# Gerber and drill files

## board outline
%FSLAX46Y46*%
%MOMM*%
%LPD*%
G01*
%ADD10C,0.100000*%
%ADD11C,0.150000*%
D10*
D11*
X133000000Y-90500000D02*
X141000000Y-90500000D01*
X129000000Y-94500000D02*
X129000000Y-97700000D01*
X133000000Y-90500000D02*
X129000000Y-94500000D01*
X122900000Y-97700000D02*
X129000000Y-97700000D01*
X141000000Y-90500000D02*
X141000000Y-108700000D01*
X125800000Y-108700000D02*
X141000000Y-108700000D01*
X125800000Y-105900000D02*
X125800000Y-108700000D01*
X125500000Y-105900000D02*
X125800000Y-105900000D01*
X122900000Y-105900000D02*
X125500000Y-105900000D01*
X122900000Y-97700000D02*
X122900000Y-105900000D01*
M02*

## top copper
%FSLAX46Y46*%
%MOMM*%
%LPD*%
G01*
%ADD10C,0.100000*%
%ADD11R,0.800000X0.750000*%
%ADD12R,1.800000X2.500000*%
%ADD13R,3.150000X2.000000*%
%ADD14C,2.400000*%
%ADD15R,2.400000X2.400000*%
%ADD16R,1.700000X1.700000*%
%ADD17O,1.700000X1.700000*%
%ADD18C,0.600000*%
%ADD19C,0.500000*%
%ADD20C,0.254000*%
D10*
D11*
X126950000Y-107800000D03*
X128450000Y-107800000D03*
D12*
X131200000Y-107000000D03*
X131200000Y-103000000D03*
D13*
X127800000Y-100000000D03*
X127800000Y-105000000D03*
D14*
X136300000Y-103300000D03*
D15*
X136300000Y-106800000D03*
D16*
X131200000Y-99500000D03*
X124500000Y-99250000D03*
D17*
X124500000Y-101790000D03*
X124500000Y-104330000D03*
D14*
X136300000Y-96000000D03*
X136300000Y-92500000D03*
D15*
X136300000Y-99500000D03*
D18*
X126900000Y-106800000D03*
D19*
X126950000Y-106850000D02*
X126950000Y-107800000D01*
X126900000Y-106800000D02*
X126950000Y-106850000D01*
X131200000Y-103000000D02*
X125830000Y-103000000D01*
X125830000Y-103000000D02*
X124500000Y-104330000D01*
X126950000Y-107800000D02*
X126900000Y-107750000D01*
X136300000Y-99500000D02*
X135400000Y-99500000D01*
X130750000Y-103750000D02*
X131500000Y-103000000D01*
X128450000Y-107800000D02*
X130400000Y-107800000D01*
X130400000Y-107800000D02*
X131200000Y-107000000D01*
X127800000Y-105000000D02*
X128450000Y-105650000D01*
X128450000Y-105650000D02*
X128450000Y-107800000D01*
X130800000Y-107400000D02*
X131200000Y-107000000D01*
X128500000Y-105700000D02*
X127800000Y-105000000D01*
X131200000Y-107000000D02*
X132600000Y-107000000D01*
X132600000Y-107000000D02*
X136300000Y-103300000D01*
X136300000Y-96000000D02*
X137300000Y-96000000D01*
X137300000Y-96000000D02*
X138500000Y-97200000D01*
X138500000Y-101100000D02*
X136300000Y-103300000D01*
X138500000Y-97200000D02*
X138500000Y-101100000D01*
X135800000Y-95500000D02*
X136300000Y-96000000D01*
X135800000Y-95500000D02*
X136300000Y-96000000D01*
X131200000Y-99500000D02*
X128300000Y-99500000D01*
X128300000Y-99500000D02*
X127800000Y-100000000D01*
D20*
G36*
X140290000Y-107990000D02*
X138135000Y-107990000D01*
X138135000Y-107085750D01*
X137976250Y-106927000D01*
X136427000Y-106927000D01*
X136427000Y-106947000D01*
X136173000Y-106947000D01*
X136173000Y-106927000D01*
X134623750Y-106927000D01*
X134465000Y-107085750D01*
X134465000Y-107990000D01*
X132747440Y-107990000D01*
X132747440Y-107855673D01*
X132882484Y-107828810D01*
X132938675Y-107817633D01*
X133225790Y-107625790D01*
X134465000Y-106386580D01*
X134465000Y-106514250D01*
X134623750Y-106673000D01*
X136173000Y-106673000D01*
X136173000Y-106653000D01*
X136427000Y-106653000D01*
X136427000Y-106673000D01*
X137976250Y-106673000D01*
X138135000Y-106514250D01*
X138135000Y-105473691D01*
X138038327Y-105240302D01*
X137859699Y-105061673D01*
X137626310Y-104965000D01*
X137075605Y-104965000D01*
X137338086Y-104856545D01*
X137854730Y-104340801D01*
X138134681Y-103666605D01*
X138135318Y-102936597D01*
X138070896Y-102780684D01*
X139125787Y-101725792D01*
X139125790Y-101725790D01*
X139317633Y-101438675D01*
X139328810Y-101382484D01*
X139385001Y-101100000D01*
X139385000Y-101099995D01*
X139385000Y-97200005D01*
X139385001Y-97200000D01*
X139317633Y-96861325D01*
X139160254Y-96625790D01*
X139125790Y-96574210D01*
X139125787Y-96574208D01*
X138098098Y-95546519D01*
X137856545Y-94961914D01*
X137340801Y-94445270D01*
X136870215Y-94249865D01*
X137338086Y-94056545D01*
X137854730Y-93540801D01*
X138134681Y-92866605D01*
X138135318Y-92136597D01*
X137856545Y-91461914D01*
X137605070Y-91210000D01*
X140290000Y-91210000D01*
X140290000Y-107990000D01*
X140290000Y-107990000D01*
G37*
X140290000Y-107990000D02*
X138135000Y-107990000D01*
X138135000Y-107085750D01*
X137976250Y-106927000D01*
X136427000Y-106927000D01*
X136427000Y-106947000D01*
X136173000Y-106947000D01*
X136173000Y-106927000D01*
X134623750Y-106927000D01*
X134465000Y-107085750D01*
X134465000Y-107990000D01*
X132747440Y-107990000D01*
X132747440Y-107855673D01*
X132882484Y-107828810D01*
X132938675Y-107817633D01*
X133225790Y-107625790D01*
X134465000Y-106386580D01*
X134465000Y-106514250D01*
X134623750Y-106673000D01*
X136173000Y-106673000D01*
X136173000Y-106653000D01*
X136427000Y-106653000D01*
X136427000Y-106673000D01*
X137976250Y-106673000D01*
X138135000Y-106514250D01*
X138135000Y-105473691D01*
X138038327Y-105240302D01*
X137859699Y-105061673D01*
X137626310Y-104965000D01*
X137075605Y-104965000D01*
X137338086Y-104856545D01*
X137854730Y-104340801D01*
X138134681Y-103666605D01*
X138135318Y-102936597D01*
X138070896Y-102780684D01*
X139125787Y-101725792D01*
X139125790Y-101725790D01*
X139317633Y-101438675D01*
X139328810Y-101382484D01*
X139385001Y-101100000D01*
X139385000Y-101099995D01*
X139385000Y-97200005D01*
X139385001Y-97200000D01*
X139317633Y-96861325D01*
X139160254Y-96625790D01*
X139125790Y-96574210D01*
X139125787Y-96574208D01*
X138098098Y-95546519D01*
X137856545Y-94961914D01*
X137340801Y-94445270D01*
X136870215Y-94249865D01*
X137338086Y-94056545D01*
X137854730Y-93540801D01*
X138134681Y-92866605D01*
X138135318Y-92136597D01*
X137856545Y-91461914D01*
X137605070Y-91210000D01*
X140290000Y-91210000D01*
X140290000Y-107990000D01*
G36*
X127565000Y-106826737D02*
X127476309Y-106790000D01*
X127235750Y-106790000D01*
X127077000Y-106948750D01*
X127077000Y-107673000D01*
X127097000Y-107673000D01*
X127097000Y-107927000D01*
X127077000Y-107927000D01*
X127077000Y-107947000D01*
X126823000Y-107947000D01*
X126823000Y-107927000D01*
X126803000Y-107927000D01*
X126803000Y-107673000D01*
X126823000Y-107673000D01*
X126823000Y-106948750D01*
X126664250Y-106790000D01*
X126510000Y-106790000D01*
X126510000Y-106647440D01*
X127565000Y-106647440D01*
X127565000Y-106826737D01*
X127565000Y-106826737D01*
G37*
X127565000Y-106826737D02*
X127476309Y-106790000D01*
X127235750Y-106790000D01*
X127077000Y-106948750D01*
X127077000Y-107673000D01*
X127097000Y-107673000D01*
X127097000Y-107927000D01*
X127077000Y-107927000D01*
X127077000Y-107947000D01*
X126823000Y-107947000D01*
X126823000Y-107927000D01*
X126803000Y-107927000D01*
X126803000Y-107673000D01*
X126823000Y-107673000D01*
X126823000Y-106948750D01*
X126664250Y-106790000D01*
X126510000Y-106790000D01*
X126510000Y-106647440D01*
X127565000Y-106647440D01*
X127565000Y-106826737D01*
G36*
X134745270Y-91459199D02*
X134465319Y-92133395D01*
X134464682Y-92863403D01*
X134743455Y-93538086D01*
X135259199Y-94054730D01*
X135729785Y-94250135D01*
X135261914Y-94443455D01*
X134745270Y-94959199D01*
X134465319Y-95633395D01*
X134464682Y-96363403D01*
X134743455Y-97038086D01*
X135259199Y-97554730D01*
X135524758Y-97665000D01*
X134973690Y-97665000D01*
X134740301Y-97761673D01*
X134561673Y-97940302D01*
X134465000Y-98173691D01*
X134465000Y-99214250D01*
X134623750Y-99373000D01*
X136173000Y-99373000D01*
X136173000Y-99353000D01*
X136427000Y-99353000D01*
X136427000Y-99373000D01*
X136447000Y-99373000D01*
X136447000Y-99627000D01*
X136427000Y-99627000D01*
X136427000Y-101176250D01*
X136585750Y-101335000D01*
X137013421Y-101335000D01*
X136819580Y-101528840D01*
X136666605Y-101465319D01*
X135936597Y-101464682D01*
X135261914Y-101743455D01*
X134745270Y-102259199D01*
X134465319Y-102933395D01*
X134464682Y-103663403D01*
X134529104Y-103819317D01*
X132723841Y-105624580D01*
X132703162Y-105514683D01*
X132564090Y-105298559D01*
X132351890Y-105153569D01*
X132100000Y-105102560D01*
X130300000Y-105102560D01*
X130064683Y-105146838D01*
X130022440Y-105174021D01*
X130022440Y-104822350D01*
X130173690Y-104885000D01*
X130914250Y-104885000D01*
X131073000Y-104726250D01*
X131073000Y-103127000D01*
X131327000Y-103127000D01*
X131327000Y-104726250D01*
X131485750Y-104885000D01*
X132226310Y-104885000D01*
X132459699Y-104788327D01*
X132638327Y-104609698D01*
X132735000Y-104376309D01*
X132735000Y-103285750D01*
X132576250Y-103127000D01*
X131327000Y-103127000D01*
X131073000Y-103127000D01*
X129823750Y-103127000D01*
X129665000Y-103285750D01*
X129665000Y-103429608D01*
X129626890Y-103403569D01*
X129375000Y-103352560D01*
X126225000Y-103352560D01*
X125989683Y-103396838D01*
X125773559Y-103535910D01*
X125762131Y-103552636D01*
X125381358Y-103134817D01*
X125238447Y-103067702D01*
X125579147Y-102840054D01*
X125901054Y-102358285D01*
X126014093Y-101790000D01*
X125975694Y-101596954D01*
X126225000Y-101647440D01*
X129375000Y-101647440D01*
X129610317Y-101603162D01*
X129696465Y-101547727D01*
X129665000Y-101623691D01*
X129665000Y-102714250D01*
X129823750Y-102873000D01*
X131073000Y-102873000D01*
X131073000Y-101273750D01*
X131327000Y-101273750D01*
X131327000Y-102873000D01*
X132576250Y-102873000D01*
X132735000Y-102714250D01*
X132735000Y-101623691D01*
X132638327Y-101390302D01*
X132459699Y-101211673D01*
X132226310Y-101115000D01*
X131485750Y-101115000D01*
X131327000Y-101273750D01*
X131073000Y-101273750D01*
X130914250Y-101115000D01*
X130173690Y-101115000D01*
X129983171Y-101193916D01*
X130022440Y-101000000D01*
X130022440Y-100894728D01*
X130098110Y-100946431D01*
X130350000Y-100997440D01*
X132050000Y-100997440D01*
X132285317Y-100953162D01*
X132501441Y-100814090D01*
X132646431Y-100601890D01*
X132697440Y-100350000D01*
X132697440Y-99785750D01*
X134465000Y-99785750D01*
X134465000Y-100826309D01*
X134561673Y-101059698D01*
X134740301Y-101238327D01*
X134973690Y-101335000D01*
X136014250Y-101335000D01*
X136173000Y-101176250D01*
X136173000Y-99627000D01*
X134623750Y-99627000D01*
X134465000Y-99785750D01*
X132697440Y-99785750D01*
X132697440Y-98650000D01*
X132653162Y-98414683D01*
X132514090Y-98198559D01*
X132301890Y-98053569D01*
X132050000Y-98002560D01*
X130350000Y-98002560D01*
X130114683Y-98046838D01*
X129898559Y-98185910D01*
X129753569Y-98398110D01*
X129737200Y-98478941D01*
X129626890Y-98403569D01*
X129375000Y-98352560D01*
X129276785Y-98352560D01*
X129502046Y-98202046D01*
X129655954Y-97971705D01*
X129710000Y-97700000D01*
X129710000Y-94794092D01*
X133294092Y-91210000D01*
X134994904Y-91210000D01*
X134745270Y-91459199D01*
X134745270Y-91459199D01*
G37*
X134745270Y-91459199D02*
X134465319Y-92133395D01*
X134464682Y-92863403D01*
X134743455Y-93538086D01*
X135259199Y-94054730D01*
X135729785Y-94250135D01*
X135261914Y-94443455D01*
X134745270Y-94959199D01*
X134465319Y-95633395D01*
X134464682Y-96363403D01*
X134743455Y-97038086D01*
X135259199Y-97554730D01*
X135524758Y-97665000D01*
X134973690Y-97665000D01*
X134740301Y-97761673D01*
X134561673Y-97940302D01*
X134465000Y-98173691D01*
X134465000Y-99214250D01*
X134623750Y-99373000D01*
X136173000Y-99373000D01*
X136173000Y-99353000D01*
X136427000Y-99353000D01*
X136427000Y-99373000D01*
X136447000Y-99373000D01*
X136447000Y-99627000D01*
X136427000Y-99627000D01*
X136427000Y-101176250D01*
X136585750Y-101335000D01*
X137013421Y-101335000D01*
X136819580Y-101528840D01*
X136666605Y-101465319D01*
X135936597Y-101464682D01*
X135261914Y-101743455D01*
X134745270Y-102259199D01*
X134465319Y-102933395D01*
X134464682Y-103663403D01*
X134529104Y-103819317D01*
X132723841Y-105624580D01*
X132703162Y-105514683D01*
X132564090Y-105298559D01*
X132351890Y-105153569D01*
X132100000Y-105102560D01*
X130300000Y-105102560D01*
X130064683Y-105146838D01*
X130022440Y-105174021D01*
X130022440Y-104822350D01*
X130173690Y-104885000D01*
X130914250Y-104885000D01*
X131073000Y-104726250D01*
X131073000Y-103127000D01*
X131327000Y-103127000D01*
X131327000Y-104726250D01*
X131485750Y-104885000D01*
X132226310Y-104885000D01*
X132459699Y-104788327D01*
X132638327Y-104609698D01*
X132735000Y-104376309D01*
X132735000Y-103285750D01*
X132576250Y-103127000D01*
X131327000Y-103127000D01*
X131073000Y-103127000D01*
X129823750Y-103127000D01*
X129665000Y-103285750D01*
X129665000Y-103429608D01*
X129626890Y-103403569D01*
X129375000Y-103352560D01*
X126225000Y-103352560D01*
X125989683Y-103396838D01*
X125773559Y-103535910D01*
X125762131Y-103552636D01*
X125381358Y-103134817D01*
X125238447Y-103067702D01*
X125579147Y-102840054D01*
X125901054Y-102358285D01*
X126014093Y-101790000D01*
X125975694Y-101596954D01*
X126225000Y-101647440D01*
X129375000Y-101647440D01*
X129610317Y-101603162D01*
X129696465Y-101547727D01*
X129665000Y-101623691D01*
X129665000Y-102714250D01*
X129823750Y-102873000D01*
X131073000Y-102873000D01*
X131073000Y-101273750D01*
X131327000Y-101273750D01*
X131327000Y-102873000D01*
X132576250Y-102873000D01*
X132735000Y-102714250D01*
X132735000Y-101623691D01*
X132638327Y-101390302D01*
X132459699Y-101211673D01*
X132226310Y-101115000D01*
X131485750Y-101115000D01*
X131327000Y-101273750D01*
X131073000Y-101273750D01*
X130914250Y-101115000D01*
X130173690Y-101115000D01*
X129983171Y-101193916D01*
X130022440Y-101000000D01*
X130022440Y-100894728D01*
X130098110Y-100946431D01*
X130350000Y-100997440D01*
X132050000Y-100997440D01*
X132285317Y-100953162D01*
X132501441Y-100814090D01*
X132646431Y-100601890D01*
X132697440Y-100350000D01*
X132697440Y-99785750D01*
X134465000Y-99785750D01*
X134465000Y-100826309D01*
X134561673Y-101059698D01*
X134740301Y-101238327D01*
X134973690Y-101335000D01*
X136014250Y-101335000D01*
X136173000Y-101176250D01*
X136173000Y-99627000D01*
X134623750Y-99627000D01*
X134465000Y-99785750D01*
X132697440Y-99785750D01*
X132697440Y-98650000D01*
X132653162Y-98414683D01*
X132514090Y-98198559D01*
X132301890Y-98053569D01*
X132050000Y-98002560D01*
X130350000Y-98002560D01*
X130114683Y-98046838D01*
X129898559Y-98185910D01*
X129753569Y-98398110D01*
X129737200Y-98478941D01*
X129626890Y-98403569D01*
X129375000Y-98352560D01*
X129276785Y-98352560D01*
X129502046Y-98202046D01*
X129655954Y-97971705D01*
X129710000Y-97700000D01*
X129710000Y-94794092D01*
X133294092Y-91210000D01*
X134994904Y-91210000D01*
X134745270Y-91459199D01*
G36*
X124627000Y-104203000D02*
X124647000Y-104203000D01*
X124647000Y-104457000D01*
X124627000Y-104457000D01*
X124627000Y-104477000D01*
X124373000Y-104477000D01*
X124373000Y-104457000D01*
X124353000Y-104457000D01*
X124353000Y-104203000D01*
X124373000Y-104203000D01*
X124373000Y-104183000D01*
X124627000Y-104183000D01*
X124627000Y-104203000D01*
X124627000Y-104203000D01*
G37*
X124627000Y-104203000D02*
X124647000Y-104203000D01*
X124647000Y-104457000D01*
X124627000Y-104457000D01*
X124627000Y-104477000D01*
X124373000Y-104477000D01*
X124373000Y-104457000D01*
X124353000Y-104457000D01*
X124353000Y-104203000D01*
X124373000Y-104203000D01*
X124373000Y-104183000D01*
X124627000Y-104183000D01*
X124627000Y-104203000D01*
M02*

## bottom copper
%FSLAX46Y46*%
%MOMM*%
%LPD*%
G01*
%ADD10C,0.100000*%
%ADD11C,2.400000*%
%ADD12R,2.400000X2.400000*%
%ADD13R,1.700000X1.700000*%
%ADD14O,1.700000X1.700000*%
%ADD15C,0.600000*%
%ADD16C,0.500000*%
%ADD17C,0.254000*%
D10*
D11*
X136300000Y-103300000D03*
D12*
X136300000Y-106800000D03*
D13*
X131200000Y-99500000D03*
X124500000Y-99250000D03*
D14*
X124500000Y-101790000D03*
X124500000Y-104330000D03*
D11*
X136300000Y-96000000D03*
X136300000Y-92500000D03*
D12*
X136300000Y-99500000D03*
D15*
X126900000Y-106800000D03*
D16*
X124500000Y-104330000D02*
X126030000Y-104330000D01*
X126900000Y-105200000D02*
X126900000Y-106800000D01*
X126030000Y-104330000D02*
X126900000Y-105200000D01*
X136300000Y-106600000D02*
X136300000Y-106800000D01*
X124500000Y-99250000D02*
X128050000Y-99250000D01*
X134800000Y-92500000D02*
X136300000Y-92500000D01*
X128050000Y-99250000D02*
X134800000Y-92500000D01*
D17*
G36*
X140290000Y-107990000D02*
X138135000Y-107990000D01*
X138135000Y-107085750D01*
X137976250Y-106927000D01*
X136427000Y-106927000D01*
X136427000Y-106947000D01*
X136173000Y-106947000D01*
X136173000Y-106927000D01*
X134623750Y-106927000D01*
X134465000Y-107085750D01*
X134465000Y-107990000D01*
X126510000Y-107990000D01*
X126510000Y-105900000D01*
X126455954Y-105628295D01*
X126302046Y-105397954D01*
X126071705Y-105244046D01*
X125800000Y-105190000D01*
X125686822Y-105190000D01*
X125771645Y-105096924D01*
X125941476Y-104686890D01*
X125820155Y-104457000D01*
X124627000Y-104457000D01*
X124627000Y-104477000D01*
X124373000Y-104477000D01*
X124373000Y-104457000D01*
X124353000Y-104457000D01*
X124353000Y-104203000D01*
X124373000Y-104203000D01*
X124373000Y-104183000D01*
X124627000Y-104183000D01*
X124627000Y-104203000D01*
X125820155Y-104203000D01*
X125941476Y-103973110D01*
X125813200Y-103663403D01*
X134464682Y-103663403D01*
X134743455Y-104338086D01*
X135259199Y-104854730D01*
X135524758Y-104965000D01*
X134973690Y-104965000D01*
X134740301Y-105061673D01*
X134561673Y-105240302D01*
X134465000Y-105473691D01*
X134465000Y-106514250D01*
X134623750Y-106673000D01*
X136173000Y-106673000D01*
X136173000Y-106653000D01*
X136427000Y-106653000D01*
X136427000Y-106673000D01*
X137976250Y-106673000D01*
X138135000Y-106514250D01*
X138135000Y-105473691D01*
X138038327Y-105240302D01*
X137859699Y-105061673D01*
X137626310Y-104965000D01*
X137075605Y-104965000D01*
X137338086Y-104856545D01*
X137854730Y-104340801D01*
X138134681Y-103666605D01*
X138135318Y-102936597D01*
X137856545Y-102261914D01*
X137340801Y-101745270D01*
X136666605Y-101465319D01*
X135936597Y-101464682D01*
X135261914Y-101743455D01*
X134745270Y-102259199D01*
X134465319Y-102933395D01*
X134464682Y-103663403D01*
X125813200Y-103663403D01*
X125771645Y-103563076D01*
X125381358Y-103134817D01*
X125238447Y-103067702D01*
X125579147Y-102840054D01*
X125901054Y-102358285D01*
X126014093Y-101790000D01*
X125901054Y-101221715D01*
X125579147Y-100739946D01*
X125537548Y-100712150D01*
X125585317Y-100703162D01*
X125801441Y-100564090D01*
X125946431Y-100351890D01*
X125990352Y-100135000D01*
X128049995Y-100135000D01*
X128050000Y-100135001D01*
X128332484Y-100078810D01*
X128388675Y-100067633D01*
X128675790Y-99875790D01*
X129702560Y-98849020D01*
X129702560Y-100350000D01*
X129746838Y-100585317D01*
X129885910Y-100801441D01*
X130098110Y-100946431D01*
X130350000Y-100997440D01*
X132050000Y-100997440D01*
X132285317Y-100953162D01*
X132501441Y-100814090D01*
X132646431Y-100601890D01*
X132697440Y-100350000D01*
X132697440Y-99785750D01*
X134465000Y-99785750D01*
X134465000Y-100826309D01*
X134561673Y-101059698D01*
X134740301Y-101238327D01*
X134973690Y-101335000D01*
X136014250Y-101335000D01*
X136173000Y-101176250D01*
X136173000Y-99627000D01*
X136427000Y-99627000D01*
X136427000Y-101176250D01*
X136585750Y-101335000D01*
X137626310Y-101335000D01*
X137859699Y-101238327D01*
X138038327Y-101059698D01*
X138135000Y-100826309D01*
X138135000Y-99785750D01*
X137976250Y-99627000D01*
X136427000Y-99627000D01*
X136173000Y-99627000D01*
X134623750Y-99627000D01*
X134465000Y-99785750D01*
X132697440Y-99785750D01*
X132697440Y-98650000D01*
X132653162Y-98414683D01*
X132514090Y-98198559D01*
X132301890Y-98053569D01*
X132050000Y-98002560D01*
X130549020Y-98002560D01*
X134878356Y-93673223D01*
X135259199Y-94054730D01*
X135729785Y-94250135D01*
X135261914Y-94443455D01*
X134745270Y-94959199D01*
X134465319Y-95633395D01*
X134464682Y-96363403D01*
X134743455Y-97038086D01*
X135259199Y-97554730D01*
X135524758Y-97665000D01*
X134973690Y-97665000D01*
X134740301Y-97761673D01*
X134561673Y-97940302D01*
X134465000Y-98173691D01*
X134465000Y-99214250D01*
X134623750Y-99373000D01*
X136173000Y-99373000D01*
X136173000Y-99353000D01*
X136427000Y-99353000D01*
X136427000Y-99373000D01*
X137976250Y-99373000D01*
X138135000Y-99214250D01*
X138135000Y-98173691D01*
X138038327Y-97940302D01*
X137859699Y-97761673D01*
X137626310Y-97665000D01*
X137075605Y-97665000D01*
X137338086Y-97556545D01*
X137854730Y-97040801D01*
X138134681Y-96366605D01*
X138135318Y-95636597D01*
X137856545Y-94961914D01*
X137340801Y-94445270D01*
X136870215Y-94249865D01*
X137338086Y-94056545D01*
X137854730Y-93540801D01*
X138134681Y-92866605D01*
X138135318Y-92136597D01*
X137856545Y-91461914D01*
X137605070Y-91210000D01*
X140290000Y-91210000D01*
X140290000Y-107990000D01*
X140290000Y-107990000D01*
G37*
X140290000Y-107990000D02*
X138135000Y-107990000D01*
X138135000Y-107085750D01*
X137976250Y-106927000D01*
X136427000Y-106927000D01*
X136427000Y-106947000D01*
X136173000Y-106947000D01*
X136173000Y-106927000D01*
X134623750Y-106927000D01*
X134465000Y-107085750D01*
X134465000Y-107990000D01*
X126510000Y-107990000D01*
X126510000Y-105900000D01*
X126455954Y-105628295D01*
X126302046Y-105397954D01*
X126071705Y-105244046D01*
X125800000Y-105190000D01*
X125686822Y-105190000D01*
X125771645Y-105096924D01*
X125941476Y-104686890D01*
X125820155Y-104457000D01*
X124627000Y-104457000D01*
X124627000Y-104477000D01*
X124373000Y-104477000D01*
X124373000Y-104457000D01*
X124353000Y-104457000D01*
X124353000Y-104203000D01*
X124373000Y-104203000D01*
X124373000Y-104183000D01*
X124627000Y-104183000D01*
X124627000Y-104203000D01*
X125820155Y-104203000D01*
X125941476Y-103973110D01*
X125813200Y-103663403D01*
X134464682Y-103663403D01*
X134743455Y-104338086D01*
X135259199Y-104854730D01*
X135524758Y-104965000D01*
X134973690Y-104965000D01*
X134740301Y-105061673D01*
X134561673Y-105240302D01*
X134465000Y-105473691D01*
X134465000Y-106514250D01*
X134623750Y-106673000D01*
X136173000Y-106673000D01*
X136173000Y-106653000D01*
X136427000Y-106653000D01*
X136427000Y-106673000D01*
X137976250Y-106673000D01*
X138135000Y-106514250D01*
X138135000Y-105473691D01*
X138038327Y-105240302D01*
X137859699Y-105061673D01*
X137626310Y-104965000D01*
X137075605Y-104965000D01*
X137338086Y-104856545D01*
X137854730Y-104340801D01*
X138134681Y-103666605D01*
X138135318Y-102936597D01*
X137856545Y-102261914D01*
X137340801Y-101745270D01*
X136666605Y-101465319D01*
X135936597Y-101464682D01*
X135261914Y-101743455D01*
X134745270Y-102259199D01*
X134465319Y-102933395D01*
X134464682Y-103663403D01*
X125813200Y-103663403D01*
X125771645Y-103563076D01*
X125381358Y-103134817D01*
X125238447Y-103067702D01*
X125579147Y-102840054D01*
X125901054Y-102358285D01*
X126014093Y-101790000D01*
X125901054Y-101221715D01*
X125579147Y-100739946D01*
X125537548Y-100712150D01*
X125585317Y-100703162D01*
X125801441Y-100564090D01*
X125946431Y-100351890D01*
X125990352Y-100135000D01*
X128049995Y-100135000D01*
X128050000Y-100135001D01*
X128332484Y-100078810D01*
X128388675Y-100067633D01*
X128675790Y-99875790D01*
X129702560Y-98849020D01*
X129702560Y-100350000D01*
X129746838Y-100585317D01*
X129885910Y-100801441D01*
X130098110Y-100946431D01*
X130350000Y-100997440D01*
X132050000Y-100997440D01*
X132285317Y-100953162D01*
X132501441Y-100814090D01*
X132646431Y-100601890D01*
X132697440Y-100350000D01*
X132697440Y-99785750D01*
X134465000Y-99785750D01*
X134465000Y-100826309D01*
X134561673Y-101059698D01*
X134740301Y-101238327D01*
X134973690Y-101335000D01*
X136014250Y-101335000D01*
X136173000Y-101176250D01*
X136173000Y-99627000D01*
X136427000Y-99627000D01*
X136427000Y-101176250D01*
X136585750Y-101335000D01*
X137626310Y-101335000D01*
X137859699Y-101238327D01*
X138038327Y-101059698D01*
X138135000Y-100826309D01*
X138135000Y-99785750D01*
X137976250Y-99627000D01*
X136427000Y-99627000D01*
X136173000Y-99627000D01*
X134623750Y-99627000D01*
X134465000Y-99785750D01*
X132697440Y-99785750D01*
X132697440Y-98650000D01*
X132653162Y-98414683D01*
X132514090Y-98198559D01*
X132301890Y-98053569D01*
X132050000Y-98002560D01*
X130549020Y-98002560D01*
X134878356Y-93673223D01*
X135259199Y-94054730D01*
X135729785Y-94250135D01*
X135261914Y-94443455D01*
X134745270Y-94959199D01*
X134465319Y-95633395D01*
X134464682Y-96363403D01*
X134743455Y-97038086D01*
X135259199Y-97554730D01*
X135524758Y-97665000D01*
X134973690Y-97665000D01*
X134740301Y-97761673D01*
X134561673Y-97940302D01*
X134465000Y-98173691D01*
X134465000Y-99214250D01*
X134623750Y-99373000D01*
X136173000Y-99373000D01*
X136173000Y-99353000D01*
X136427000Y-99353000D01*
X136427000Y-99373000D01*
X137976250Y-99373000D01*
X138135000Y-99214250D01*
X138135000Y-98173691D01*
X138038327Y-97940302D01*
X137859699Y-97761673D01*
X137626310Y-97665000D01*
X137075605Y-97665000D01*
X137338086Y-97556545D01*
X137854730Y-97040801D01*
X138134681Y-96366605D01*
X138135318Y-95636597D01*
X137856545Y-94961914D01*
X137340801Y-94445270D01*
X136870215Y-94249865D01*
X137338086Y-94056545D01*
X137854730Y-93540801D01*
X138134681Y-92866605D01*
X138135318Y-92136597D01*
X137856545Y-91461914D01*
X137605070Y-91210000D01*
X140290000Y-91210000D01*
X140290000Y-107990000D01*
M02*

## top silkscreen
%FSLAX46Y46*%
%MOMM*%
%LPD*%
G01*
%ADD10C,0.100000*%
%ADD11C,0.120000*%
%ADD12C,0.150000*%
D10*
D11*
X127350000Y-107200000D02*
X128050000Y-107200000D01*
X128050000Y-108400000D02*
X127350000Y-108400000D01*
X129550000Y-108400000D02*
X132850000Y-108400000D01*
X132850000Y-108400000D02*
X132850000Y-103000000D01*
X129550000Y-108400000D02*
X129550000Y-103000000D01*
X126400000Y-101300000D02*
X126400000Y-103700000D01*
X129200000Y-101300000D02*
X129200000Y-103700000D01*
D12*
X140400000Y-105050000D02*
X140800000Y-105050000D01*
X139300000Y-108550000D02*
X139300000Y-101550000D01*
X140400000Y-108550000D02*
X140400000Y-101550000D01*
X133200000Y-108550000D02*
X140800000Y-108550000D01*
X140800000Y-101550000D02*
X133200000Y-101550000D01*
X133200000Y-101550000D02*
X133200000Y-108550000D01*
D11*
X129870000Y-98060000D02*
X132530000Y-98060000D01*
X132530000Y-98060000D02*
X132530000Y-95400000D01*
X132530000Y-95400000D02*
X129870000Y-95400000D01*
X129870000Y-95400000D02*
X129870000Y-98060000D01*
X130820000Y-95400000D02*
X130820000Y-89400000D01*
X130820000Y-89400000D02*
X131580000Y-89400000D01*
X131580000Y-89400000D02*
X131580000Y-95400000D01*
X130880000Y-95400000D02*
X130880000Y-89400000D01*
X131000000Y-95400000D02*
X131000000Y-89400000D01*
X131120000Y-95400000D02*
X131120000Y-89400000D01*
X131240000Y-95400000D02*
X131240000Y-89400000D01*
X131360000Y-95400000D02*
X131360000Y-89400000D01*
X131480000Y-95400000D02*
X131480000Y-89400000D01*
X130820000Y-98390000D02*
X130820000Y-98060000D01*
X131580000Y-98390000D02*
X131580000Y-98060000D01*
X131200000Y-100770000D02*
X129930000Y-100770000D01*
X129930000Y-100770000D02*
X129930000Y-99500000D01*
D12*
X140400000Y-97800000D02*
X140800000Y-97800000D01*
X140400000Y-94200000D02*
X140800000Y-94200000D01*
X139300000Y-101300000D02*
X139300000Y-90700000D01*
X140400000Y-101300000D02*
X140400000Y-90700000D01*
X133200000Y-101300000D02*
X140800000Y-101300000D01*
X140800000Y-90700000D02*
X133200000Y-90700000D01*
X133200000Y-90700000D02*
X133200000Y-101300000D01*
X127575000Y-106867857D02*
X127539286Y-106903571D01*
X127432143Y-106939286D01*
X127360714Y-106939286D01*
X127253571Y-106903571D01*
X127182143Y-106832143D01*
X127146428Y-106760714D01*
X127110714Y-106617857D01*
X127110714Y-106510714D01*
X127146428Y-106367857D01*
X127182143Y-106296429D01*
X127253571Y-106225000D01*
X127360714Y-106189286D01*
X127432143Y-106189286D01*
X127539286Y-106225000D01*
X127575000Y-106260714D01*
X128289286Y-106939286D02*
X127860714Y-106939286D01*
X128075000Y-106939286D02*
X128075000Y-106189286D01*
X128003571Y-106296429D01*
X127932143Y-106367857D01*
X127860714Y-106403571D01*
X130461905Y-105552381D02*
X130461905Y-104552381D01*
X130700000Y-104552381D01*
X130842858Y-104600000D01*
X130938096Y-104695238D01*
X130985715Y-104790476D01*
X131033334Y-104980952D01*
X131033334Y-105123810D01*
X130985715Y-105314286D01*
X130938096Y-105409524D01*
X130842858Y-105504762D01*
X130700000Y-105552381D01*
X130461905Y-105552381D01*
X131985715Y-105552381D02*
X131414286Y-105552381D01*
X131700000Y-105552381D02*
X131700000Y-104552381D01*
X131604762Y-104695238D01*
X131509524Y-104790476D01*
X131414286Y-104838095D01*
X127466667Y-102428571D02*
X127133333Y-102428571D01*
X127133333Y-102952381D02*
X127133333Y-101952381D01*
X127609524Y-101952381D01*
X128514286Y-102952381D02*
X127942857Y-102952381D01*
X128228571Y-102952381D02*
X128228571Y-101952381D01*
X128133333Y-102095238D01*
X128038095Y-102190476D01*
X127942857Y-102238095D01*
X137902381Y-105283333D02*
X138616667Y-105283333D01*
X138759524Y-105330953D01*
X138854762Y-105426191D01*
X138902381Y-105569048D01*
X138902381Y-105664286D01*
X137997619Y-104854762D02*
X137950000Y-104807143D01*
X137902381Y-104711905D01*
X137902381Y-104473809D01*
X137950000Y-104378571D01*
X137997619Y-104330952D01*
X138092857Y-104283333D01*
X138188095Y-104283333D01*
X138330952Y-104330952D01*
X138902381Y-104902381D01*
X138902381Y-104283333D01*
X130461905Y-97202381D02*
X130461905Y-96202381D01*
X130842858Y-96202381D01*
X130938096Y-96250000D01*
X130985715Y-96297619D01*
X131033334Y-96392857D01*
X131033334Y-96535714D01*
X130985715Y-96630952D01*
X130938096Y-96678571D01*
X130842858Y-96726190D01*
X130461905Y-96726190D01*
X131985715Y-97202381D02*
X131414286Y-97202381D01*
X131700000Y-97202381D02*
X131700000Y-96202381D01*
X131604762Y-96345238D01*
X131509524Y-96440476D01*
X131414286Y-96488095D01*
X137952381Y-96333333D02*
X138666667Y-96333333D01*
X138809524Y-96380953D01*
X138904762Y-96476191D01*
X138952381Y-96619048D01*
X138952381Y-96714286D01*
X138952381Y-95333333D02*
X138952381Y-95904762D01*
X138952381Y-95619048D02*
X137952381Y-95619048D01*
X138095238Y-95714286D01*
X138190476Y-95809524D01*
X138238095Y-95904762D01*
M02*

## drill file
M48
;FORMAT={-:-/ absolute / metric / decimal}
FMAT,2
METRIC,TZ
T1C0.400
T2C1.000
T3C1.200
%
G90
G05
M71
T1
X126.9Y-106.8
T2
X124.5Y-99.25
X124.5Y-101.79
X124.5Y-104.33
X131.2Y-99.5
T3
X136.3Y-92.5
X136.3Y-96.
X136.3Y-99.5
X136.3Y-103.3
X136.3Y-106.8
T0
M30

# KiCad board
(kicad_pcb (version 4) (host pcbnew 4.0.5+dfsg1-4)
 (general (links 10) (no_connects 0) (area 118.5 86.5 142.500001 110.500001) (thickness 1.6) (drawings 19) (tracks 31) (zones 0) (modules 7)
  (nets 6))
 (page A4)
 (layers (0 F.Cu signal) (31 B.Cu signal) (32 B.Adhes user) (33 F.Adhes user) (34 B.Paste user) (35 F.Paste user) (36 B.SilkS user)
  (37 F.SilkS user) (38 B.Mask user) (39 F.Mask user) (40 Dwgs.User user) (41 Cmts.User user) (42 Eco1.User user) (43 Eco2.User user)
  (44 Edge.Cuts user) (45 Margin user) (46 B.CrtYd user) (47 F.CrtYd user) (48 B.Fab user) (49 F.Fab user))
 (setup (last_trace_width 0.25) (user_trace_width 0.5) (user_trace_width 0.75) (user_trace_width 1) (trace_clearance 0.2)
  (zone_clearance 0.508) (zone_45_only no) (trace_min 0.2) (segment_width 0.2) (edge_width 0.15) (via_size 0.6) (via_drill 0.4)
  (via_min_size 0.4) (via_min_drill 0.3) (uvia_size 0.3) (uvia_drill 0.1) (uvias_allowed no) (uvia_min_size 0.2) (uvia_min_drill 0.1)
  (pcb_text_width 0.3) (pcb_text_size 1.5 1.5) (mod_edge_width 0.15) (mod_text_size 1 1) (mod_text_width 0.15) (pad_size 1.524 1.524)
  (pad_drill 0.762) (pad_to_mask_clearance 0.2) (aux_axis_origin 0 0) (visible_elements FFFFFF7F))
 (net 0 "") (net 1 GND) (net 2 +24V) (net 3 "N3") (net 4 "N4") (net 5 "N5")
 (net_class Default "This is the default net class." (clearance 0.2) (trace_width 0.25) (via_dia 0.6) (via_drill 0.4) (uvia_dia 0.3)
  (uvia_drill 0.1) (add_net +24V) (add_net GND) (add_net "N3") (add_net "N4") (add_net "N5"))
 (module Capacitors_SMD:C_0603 (layer F.Cu) (at 127.7 107.8 180)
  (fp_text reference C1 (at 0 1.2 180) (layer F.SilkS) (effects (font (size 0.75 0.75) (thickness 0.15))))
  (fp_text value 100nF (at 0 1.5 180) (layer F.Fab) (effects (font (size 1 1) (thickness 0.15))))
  (fp_line (start 0.35 0.6) (end -0.35 0.6) (layer F.SilkS) (width 0.12))
  (fp_line (start -0.35 -0.6) (end 0.35 -0.6) (layer F.SilkS) (width 0.12))
  (pad 2 smd rect (at 0.75 0 180) (size 0.8 0.75) (layers F.Cu F.Paste F.Mask) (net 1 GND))
  (pad 1 smd rect (at -0.75 0 180) (size 0.8 0.75) (layers F.Cu F.Paste F.Mask) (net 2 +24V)))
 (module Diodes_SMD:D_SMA (layer F.Cu) (at 131.2 105 90)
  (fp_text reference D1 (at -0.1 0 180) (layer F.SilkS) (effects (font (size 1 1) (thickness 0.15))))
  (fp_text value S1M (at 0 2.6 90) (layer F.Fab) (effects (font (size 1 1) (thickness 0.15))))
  (fp_line (start -3.4 -1.65) (end -3.4 1.65) (layer F.SilkS) (width 0.12))
  (fp_line (start -3.4 1.65) (end 2 1.65) (layer F.SilkS) (width 0.12))
  (fp_line (start -3.4 -1.65) (end 2 -1.65) (layer F.SilkS) (width 0.12))
  (pad 1 smd rect (at -2 0 90) (size 2.5 1.8) (layers F.Cu F.Paste F.Mask) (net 2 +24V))
  (pad 2 smd rect (at 2 0 90) (size 2.5 1.8) (layers F.Cu F.Paste F.Mask) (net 1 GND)))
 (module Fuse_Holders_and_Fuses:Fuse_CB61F (layer F.Cu) (at 127.8 102.5 270)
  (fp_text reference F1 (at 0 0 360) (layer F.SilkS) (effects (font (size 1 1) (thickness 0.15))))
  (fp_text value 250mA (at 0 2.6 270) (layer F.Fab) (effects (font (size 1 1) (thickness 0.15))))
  (fp_line (start -1.2 1.4) (end 1.2 1.4) (layer F.SilkS) (width 0.12))
  (fp_line (start -1.2 -1.4) (end 1.2 -1.4) (layer F.SilkS) (width 0.12))
  (pad 1 smd rect (at -2.5 0 270) (size 2 3.15) (layers F.Cu F.Paste F.Mask) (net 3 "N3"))
  (pad 2 smd rect (at 2.5 0 270) (size 2 3.15) (layers F.Cu F.Paste F.Mask) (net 2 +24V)))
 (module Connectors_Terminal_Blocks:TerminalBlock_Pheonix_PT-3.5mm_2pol (layer F.Cu) (at 136.3 106.8 90)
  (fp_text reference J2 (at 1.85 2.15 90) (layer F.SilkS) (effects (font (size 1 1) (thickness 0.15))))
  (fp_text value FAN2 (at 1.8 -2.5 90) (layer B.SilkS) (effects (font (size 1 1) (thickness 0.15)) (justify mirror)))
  (fp_line (start 1.75 4.1) (end 1.75 4.5) (layer F.SilkS) (width 0.15))
  (fp_line (start -1.75 3) (end 5.25 3) (layer F.SilkS) (width 0.15))
  (fp_line (start -1.75 4.1) (end 5.25 4.1) (layer F.SilkS) (width 0.15))
  (fp_line (start -1.75 -3.1) (end -1.75 4.5) (layer F.SilkS) (width 0.15))
  (fp_line (start 5.25 4.5) (end 5.25 -3.1) (layer F.SilkS) (width 0.15))
  (fp_line (start 5.25 -3.1) (end -1.75 -3.1) (layer F.SilkS) (width 0.15))
  (pad 2 thru_hole circle (at 3.5 0 90) (size 2.4 2.4) (drill 1.2) (layers *.Cu *.Mask) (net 2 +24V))
  (pad 1 thru_hole rect (at 0 0 90) (size 2.4 2.4) (drill 1.2) (layers *.Cu *.Mask) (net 1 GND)))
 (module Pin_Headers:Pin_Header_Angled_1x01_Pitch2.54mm (layer F.Cu) (at 131.2 99.5 90)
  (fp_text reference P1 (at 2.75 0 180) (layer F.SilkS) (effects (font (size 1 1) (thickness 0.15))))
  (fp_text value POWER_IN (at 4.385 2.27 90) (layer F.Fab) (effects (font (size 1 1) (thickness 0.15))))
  (fp_line (start 1.44 -1.33) (end 1.44 1.33) (layer F.SilkS) (width 0.12))
  (fp_line (start 1.44 1.33) (end 4.1 1.33) (layer F.SilkS) (width 0.12))
  (fp_line (start 4.1 1.33) (end 4.1 -1.33) (layer F.SilkS) (width 0.12))
  (fp_line (start 4.1 -1.33) (end 1.44 -1.33) (layer F.SilkS) (width 0.12))
  (fp_line (start 4.1 -0.38) (end 10.1 -0.38) (layer F.SilkS) (width 0.12))
  (fp_line (start 10.1 -0.38) (end 10.1 0.38) (layer F.SilkS) (width 0.12))
  (fp_line (start 10.1 0.38) (end 4.1 0.38) (layer F.SilkS) (width 0.12))
  (fp_line (start 4.1 -0.32) (end 10.1 -0.32) (layer F.SilkS) (width 0.12))
  (fp_line (start 4.1 -0.2) (end 10.1 -0.2) (layer F.SilkS) (width 0.12))
  (fp_line (start 4.1 -0.08) (end 10.1 -0.08) (layer F.SilkS) (width 0.12))
  (fp_line (start 4.1 0.04) (end 10.1 0.04) (layer F.SilkS) (width 0.12))
  (fp_line (start 4.1 0.16) (end 10.1 0.16) (layer F.SilkS) (width 0.12))
  (fp_line (start 4.1 0.28) (end 10.1 0.28) (layer F.SilkS) (width 0.12))
  (fp_line (start 1.11 -0.38) (end 1.44 -0.38) (layer F.SilkS) (width 0.12))
  (fp_line (start 1.11 0.38) (end 1.44 0.38) (layer F.SilkS) (width 0.12))
  (fp_line (start -1.27 0) (end -1.27 -1.27) (layer F.SilkS) (width 0.12))
  (fp_line (start -1.27 -1.27) (end 0 -1.27) (layer F.SilkS) (width 0.12))
  (pad 1 thru_hole rect (at 0 0 90) (size 1.7 1.7) (drill 1) (layers *.Cu *.Mask) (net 3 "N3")))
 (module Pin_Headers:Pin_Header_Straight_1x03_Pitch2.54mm (layer B.Cu) (at 124.5 99.25 180)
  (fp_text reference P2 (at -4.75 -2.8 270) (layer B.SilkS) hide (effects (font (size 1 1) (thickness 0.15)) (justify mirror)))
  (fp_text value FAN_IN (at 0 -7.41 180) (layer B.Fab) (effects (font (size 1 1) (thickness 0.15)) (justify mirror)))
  (pad 1 thru_hole rect (at 0 0 180) (size 1.7 1.7) (drill 1) (layers *.Cu *.Mask) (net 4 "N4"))
  (pad 2 thru_hole oval (at 0 -2.54 180) (size 1.7 1.7) (drill 1) (layers *.Cu *.Mask) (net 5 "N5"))
  (pad 3 thru_hole oval (at 0 -5.08 180) (size 1.7 1.7) (drill 1) (layers *.Cu *.Mask) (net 1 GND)))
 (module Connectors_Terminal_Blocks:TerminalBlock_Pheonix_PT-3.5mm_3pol (layer F.Cu) (at 136.3 99.5 90)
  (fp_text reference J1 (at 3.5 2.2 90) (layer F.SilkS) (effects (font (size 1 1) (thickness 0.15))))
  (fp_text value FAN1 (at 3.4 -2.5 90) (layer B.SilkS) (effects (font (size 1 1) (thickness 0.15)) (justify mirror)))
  (fp_line (start 1.7 4.1) (end 1.7 4.5) (layer F.SilkS) (width 0.15))
  (fp_line (start 5.3 4.1) (end 5.3 4.5) (layer F.SilkS) (width 0.15))
  (fp_line (start -1.8 3) (end 8.8 3) (layer F.SilkS) (width 0.15))
  (fp_line (start -1.8 4.1) (end 8.8 4.1) (layer F.SilkS) (width 0.15))
  (fp_line (start -1.8 -3.1) (end -1.8 4.5) (layer F.SilkS) (width 0.15))
  (fp_line (start 8.8 4.5) (end 8.8 -3.1) (layer F.SilkS) (width 0.15))
  (fp_line (start 8.8 -3.1) (end -1.8 -3.1) (layer F.SilkS) (width 0.15))
  (pad 2 thru_hole circle (at 3.5 0 90) (size 2.4 2.4) (drill 1.2) (layers *.Cu *.Mask) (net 2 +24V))
  (pad 3 thru_hole circle (at 7 0 90) (size 2.4 2.4) (drill 1.2) (layers *.Cu *.Mask) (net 4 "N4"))
  (pad 1 thru_hole rect (at 0 0 90) (size 2.4 2.4) (drill 1.2) (layers *.Cu *.Mask) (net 1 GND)))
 (gr_line (start 133 90.5) (end 141 90.5) (angle 90) (layer Edge.Cuts) (width 0.15))
 (gr_line (start 129 94.5) (end 129 97.7) (angle 90) (layer Edge.Cuts) (width 0.15))
 (gr_line (start 133 90.5) (end 129 94.5) (angle 90) (layer Edge.Cuts) (width 0.15))
 (gr_line (start 122.9 97.7) (end 129 97.7) (angle 90) (layer Edge.Cuts) (width 0.15))
 (gr_line (start 141 90.5) (end 141 108.7) (angle 90) (layer Edge.Cuts) (width 0.15))
 (gr_line (start 125.8 108.7) (end 141 108.7) (angle 90) (layer Edge.Cuts) (width 0.15))
 (gr_line (start 125.8 105.9) (end 125.8 108.7) (angle 90) (layer Edge.Cuts) (width 0.15))
 (gr_line (start 125.5 105.9) (end 125.8 105.9) (angle 90) (layer Edge.Cuts) (width 0.15))
 (gr_line (start 122.9 105.9) (end 125.5 105.9) (angle 90) (layer Edge.Cuts) (width 0.15))
 (gr_line (start 122.9 97.7) (end 122.9 105.9) (angle 90) (layer Edge.Cuts) (width 0.15))
 (segment (start 124.5 104.33) (end 126.03 104.33) (width 0.5) (layer B.Cu) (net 1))
 (segment (start 126.95 106.85) (end 126.95 107.8) (width 0.5) (layer F.Cu) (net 1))
 (segment (start 126.9 106.8) (end 126.95 106.85) (width 0.5) (layer F.Cu) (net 1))
 (via (at 126.9 106.8) (size 0.6) (drill 0.4) (layers F.Cu B.Cu) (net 1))
 (segment (start 126.9 105.2) (end 126.9 106.8) (width 0.5) (layer B.Cu) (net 1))
 (segment (start 126.03 104.33) (end 126.9 105.2) (width 0.5) (layer B.Cu) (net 1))
 (segment (start 131.2 103) (end 125.83 103) (width 0.5) (layer F.Cu) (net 1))
 (segment (start 125.83 103) (end 124.5 104.33) (width 0.5) (layer F.Cu) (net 1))
 (segment (start 126.95 107.8) (end 126.9 107.75) (width 0.5) (layer F.Cu) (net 1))
 (segment (start 136.3 99.5) (end 135.4 99.5) (width 0.5) (layer F.Cu) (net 1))
 (segment (start 136.3 106.6) (end 136.3 106.8) (width 0.5) (layer B.Cu) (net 1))
 (segment (start 130.75 103.75) (end 131.5 103) (width 0.5) (layer F.Cu) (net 1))
 (segment (start 128.45 107.8) (end 130.4 107.8) (width 0.5) (layer F.Cu) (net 2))
 (segment (start 130.4 107.8) (end 131.2 107) (width 0.5) (layer F.Cu) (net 2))
 (segment (start 127.8 105) (end 128.45 105.65) (width 0.5) (layer F.Cu) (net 2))
 (segment (start 128.45 105.65) (end 128.45 107.8) (width 0.5) (layer F.Cu) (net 2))
 (segment (start 130.8 107.4) (end 131.2 107) (width 0.5) (layer F.Cu) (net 2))
 (segment (start 128.5 105.7) (end 127.8 105) (width 0.5) (layer F.Cu) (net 2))
 (segment (start 131.2 107) (end 132.6 107) (width 0.5) (layer F.Cu) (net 2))
 (segment (start 132.6 107) (end 136.3 103.3) (width 0.5) (layer F.Cu) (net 2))
 (segment (start 136.3 96) (end 137.3 96) (width 0.5) (layer F.Cu) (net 2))
 (segment (start 137.3 96) (end 138.5 97.2) (width 0.5) (layer F.Cu) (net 2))
 (segment (start 138.5 101.1) (end 136.3 103.3) (width 0.5) (layer F.Cu) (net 2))
 (segment (start 138.5 97.2) (end 138.5 101.1) (width 0.5) (layer F.Cu) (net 2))
 (segment (start 135.8 95.5) (end 136.3 96) (width 0.5) (layer F.Cu) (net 2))
 (segment (start 135.8 95.5) (end 136.3 96) (width 0.5) (layer F.Cu) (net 2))
 (segment (start 131.2 99.5) (end 128.3 99.5) (width 0.5) (layer F.Cu) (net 3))
 (segment (start 128.3 99.5) (end 127.8 100) (width 0.5) (layer F.Cu) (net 3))
 (segment (start 124.5 99.25) (end 128.05 99.25) (width 0.5) (layer B.Cu) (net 4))
 (segment (start 134.8 92.5) (end 136.3 92.5) (width 0.5) (layer B.Cu) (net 4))
 (segment (start 128.05 99.25) (end 134.8 92.5) (width 0.5) (layer B.Cu) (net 4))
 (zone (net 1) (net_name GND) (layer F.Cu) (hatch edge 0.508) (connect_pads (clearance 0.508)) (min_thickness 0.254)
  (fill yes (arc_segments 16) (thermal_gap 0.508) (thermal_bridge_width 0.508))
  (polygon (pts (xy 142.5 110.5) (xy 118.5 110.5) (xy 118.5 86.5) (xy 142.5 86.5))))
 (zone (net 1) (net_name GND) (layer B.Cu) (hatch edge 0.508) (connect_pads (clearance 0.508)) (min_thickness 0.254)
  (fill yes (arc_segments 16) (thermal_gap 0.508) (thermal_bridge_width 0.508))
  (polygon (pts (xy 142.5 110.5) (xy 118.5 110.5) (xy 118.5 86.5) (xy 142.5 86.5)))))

